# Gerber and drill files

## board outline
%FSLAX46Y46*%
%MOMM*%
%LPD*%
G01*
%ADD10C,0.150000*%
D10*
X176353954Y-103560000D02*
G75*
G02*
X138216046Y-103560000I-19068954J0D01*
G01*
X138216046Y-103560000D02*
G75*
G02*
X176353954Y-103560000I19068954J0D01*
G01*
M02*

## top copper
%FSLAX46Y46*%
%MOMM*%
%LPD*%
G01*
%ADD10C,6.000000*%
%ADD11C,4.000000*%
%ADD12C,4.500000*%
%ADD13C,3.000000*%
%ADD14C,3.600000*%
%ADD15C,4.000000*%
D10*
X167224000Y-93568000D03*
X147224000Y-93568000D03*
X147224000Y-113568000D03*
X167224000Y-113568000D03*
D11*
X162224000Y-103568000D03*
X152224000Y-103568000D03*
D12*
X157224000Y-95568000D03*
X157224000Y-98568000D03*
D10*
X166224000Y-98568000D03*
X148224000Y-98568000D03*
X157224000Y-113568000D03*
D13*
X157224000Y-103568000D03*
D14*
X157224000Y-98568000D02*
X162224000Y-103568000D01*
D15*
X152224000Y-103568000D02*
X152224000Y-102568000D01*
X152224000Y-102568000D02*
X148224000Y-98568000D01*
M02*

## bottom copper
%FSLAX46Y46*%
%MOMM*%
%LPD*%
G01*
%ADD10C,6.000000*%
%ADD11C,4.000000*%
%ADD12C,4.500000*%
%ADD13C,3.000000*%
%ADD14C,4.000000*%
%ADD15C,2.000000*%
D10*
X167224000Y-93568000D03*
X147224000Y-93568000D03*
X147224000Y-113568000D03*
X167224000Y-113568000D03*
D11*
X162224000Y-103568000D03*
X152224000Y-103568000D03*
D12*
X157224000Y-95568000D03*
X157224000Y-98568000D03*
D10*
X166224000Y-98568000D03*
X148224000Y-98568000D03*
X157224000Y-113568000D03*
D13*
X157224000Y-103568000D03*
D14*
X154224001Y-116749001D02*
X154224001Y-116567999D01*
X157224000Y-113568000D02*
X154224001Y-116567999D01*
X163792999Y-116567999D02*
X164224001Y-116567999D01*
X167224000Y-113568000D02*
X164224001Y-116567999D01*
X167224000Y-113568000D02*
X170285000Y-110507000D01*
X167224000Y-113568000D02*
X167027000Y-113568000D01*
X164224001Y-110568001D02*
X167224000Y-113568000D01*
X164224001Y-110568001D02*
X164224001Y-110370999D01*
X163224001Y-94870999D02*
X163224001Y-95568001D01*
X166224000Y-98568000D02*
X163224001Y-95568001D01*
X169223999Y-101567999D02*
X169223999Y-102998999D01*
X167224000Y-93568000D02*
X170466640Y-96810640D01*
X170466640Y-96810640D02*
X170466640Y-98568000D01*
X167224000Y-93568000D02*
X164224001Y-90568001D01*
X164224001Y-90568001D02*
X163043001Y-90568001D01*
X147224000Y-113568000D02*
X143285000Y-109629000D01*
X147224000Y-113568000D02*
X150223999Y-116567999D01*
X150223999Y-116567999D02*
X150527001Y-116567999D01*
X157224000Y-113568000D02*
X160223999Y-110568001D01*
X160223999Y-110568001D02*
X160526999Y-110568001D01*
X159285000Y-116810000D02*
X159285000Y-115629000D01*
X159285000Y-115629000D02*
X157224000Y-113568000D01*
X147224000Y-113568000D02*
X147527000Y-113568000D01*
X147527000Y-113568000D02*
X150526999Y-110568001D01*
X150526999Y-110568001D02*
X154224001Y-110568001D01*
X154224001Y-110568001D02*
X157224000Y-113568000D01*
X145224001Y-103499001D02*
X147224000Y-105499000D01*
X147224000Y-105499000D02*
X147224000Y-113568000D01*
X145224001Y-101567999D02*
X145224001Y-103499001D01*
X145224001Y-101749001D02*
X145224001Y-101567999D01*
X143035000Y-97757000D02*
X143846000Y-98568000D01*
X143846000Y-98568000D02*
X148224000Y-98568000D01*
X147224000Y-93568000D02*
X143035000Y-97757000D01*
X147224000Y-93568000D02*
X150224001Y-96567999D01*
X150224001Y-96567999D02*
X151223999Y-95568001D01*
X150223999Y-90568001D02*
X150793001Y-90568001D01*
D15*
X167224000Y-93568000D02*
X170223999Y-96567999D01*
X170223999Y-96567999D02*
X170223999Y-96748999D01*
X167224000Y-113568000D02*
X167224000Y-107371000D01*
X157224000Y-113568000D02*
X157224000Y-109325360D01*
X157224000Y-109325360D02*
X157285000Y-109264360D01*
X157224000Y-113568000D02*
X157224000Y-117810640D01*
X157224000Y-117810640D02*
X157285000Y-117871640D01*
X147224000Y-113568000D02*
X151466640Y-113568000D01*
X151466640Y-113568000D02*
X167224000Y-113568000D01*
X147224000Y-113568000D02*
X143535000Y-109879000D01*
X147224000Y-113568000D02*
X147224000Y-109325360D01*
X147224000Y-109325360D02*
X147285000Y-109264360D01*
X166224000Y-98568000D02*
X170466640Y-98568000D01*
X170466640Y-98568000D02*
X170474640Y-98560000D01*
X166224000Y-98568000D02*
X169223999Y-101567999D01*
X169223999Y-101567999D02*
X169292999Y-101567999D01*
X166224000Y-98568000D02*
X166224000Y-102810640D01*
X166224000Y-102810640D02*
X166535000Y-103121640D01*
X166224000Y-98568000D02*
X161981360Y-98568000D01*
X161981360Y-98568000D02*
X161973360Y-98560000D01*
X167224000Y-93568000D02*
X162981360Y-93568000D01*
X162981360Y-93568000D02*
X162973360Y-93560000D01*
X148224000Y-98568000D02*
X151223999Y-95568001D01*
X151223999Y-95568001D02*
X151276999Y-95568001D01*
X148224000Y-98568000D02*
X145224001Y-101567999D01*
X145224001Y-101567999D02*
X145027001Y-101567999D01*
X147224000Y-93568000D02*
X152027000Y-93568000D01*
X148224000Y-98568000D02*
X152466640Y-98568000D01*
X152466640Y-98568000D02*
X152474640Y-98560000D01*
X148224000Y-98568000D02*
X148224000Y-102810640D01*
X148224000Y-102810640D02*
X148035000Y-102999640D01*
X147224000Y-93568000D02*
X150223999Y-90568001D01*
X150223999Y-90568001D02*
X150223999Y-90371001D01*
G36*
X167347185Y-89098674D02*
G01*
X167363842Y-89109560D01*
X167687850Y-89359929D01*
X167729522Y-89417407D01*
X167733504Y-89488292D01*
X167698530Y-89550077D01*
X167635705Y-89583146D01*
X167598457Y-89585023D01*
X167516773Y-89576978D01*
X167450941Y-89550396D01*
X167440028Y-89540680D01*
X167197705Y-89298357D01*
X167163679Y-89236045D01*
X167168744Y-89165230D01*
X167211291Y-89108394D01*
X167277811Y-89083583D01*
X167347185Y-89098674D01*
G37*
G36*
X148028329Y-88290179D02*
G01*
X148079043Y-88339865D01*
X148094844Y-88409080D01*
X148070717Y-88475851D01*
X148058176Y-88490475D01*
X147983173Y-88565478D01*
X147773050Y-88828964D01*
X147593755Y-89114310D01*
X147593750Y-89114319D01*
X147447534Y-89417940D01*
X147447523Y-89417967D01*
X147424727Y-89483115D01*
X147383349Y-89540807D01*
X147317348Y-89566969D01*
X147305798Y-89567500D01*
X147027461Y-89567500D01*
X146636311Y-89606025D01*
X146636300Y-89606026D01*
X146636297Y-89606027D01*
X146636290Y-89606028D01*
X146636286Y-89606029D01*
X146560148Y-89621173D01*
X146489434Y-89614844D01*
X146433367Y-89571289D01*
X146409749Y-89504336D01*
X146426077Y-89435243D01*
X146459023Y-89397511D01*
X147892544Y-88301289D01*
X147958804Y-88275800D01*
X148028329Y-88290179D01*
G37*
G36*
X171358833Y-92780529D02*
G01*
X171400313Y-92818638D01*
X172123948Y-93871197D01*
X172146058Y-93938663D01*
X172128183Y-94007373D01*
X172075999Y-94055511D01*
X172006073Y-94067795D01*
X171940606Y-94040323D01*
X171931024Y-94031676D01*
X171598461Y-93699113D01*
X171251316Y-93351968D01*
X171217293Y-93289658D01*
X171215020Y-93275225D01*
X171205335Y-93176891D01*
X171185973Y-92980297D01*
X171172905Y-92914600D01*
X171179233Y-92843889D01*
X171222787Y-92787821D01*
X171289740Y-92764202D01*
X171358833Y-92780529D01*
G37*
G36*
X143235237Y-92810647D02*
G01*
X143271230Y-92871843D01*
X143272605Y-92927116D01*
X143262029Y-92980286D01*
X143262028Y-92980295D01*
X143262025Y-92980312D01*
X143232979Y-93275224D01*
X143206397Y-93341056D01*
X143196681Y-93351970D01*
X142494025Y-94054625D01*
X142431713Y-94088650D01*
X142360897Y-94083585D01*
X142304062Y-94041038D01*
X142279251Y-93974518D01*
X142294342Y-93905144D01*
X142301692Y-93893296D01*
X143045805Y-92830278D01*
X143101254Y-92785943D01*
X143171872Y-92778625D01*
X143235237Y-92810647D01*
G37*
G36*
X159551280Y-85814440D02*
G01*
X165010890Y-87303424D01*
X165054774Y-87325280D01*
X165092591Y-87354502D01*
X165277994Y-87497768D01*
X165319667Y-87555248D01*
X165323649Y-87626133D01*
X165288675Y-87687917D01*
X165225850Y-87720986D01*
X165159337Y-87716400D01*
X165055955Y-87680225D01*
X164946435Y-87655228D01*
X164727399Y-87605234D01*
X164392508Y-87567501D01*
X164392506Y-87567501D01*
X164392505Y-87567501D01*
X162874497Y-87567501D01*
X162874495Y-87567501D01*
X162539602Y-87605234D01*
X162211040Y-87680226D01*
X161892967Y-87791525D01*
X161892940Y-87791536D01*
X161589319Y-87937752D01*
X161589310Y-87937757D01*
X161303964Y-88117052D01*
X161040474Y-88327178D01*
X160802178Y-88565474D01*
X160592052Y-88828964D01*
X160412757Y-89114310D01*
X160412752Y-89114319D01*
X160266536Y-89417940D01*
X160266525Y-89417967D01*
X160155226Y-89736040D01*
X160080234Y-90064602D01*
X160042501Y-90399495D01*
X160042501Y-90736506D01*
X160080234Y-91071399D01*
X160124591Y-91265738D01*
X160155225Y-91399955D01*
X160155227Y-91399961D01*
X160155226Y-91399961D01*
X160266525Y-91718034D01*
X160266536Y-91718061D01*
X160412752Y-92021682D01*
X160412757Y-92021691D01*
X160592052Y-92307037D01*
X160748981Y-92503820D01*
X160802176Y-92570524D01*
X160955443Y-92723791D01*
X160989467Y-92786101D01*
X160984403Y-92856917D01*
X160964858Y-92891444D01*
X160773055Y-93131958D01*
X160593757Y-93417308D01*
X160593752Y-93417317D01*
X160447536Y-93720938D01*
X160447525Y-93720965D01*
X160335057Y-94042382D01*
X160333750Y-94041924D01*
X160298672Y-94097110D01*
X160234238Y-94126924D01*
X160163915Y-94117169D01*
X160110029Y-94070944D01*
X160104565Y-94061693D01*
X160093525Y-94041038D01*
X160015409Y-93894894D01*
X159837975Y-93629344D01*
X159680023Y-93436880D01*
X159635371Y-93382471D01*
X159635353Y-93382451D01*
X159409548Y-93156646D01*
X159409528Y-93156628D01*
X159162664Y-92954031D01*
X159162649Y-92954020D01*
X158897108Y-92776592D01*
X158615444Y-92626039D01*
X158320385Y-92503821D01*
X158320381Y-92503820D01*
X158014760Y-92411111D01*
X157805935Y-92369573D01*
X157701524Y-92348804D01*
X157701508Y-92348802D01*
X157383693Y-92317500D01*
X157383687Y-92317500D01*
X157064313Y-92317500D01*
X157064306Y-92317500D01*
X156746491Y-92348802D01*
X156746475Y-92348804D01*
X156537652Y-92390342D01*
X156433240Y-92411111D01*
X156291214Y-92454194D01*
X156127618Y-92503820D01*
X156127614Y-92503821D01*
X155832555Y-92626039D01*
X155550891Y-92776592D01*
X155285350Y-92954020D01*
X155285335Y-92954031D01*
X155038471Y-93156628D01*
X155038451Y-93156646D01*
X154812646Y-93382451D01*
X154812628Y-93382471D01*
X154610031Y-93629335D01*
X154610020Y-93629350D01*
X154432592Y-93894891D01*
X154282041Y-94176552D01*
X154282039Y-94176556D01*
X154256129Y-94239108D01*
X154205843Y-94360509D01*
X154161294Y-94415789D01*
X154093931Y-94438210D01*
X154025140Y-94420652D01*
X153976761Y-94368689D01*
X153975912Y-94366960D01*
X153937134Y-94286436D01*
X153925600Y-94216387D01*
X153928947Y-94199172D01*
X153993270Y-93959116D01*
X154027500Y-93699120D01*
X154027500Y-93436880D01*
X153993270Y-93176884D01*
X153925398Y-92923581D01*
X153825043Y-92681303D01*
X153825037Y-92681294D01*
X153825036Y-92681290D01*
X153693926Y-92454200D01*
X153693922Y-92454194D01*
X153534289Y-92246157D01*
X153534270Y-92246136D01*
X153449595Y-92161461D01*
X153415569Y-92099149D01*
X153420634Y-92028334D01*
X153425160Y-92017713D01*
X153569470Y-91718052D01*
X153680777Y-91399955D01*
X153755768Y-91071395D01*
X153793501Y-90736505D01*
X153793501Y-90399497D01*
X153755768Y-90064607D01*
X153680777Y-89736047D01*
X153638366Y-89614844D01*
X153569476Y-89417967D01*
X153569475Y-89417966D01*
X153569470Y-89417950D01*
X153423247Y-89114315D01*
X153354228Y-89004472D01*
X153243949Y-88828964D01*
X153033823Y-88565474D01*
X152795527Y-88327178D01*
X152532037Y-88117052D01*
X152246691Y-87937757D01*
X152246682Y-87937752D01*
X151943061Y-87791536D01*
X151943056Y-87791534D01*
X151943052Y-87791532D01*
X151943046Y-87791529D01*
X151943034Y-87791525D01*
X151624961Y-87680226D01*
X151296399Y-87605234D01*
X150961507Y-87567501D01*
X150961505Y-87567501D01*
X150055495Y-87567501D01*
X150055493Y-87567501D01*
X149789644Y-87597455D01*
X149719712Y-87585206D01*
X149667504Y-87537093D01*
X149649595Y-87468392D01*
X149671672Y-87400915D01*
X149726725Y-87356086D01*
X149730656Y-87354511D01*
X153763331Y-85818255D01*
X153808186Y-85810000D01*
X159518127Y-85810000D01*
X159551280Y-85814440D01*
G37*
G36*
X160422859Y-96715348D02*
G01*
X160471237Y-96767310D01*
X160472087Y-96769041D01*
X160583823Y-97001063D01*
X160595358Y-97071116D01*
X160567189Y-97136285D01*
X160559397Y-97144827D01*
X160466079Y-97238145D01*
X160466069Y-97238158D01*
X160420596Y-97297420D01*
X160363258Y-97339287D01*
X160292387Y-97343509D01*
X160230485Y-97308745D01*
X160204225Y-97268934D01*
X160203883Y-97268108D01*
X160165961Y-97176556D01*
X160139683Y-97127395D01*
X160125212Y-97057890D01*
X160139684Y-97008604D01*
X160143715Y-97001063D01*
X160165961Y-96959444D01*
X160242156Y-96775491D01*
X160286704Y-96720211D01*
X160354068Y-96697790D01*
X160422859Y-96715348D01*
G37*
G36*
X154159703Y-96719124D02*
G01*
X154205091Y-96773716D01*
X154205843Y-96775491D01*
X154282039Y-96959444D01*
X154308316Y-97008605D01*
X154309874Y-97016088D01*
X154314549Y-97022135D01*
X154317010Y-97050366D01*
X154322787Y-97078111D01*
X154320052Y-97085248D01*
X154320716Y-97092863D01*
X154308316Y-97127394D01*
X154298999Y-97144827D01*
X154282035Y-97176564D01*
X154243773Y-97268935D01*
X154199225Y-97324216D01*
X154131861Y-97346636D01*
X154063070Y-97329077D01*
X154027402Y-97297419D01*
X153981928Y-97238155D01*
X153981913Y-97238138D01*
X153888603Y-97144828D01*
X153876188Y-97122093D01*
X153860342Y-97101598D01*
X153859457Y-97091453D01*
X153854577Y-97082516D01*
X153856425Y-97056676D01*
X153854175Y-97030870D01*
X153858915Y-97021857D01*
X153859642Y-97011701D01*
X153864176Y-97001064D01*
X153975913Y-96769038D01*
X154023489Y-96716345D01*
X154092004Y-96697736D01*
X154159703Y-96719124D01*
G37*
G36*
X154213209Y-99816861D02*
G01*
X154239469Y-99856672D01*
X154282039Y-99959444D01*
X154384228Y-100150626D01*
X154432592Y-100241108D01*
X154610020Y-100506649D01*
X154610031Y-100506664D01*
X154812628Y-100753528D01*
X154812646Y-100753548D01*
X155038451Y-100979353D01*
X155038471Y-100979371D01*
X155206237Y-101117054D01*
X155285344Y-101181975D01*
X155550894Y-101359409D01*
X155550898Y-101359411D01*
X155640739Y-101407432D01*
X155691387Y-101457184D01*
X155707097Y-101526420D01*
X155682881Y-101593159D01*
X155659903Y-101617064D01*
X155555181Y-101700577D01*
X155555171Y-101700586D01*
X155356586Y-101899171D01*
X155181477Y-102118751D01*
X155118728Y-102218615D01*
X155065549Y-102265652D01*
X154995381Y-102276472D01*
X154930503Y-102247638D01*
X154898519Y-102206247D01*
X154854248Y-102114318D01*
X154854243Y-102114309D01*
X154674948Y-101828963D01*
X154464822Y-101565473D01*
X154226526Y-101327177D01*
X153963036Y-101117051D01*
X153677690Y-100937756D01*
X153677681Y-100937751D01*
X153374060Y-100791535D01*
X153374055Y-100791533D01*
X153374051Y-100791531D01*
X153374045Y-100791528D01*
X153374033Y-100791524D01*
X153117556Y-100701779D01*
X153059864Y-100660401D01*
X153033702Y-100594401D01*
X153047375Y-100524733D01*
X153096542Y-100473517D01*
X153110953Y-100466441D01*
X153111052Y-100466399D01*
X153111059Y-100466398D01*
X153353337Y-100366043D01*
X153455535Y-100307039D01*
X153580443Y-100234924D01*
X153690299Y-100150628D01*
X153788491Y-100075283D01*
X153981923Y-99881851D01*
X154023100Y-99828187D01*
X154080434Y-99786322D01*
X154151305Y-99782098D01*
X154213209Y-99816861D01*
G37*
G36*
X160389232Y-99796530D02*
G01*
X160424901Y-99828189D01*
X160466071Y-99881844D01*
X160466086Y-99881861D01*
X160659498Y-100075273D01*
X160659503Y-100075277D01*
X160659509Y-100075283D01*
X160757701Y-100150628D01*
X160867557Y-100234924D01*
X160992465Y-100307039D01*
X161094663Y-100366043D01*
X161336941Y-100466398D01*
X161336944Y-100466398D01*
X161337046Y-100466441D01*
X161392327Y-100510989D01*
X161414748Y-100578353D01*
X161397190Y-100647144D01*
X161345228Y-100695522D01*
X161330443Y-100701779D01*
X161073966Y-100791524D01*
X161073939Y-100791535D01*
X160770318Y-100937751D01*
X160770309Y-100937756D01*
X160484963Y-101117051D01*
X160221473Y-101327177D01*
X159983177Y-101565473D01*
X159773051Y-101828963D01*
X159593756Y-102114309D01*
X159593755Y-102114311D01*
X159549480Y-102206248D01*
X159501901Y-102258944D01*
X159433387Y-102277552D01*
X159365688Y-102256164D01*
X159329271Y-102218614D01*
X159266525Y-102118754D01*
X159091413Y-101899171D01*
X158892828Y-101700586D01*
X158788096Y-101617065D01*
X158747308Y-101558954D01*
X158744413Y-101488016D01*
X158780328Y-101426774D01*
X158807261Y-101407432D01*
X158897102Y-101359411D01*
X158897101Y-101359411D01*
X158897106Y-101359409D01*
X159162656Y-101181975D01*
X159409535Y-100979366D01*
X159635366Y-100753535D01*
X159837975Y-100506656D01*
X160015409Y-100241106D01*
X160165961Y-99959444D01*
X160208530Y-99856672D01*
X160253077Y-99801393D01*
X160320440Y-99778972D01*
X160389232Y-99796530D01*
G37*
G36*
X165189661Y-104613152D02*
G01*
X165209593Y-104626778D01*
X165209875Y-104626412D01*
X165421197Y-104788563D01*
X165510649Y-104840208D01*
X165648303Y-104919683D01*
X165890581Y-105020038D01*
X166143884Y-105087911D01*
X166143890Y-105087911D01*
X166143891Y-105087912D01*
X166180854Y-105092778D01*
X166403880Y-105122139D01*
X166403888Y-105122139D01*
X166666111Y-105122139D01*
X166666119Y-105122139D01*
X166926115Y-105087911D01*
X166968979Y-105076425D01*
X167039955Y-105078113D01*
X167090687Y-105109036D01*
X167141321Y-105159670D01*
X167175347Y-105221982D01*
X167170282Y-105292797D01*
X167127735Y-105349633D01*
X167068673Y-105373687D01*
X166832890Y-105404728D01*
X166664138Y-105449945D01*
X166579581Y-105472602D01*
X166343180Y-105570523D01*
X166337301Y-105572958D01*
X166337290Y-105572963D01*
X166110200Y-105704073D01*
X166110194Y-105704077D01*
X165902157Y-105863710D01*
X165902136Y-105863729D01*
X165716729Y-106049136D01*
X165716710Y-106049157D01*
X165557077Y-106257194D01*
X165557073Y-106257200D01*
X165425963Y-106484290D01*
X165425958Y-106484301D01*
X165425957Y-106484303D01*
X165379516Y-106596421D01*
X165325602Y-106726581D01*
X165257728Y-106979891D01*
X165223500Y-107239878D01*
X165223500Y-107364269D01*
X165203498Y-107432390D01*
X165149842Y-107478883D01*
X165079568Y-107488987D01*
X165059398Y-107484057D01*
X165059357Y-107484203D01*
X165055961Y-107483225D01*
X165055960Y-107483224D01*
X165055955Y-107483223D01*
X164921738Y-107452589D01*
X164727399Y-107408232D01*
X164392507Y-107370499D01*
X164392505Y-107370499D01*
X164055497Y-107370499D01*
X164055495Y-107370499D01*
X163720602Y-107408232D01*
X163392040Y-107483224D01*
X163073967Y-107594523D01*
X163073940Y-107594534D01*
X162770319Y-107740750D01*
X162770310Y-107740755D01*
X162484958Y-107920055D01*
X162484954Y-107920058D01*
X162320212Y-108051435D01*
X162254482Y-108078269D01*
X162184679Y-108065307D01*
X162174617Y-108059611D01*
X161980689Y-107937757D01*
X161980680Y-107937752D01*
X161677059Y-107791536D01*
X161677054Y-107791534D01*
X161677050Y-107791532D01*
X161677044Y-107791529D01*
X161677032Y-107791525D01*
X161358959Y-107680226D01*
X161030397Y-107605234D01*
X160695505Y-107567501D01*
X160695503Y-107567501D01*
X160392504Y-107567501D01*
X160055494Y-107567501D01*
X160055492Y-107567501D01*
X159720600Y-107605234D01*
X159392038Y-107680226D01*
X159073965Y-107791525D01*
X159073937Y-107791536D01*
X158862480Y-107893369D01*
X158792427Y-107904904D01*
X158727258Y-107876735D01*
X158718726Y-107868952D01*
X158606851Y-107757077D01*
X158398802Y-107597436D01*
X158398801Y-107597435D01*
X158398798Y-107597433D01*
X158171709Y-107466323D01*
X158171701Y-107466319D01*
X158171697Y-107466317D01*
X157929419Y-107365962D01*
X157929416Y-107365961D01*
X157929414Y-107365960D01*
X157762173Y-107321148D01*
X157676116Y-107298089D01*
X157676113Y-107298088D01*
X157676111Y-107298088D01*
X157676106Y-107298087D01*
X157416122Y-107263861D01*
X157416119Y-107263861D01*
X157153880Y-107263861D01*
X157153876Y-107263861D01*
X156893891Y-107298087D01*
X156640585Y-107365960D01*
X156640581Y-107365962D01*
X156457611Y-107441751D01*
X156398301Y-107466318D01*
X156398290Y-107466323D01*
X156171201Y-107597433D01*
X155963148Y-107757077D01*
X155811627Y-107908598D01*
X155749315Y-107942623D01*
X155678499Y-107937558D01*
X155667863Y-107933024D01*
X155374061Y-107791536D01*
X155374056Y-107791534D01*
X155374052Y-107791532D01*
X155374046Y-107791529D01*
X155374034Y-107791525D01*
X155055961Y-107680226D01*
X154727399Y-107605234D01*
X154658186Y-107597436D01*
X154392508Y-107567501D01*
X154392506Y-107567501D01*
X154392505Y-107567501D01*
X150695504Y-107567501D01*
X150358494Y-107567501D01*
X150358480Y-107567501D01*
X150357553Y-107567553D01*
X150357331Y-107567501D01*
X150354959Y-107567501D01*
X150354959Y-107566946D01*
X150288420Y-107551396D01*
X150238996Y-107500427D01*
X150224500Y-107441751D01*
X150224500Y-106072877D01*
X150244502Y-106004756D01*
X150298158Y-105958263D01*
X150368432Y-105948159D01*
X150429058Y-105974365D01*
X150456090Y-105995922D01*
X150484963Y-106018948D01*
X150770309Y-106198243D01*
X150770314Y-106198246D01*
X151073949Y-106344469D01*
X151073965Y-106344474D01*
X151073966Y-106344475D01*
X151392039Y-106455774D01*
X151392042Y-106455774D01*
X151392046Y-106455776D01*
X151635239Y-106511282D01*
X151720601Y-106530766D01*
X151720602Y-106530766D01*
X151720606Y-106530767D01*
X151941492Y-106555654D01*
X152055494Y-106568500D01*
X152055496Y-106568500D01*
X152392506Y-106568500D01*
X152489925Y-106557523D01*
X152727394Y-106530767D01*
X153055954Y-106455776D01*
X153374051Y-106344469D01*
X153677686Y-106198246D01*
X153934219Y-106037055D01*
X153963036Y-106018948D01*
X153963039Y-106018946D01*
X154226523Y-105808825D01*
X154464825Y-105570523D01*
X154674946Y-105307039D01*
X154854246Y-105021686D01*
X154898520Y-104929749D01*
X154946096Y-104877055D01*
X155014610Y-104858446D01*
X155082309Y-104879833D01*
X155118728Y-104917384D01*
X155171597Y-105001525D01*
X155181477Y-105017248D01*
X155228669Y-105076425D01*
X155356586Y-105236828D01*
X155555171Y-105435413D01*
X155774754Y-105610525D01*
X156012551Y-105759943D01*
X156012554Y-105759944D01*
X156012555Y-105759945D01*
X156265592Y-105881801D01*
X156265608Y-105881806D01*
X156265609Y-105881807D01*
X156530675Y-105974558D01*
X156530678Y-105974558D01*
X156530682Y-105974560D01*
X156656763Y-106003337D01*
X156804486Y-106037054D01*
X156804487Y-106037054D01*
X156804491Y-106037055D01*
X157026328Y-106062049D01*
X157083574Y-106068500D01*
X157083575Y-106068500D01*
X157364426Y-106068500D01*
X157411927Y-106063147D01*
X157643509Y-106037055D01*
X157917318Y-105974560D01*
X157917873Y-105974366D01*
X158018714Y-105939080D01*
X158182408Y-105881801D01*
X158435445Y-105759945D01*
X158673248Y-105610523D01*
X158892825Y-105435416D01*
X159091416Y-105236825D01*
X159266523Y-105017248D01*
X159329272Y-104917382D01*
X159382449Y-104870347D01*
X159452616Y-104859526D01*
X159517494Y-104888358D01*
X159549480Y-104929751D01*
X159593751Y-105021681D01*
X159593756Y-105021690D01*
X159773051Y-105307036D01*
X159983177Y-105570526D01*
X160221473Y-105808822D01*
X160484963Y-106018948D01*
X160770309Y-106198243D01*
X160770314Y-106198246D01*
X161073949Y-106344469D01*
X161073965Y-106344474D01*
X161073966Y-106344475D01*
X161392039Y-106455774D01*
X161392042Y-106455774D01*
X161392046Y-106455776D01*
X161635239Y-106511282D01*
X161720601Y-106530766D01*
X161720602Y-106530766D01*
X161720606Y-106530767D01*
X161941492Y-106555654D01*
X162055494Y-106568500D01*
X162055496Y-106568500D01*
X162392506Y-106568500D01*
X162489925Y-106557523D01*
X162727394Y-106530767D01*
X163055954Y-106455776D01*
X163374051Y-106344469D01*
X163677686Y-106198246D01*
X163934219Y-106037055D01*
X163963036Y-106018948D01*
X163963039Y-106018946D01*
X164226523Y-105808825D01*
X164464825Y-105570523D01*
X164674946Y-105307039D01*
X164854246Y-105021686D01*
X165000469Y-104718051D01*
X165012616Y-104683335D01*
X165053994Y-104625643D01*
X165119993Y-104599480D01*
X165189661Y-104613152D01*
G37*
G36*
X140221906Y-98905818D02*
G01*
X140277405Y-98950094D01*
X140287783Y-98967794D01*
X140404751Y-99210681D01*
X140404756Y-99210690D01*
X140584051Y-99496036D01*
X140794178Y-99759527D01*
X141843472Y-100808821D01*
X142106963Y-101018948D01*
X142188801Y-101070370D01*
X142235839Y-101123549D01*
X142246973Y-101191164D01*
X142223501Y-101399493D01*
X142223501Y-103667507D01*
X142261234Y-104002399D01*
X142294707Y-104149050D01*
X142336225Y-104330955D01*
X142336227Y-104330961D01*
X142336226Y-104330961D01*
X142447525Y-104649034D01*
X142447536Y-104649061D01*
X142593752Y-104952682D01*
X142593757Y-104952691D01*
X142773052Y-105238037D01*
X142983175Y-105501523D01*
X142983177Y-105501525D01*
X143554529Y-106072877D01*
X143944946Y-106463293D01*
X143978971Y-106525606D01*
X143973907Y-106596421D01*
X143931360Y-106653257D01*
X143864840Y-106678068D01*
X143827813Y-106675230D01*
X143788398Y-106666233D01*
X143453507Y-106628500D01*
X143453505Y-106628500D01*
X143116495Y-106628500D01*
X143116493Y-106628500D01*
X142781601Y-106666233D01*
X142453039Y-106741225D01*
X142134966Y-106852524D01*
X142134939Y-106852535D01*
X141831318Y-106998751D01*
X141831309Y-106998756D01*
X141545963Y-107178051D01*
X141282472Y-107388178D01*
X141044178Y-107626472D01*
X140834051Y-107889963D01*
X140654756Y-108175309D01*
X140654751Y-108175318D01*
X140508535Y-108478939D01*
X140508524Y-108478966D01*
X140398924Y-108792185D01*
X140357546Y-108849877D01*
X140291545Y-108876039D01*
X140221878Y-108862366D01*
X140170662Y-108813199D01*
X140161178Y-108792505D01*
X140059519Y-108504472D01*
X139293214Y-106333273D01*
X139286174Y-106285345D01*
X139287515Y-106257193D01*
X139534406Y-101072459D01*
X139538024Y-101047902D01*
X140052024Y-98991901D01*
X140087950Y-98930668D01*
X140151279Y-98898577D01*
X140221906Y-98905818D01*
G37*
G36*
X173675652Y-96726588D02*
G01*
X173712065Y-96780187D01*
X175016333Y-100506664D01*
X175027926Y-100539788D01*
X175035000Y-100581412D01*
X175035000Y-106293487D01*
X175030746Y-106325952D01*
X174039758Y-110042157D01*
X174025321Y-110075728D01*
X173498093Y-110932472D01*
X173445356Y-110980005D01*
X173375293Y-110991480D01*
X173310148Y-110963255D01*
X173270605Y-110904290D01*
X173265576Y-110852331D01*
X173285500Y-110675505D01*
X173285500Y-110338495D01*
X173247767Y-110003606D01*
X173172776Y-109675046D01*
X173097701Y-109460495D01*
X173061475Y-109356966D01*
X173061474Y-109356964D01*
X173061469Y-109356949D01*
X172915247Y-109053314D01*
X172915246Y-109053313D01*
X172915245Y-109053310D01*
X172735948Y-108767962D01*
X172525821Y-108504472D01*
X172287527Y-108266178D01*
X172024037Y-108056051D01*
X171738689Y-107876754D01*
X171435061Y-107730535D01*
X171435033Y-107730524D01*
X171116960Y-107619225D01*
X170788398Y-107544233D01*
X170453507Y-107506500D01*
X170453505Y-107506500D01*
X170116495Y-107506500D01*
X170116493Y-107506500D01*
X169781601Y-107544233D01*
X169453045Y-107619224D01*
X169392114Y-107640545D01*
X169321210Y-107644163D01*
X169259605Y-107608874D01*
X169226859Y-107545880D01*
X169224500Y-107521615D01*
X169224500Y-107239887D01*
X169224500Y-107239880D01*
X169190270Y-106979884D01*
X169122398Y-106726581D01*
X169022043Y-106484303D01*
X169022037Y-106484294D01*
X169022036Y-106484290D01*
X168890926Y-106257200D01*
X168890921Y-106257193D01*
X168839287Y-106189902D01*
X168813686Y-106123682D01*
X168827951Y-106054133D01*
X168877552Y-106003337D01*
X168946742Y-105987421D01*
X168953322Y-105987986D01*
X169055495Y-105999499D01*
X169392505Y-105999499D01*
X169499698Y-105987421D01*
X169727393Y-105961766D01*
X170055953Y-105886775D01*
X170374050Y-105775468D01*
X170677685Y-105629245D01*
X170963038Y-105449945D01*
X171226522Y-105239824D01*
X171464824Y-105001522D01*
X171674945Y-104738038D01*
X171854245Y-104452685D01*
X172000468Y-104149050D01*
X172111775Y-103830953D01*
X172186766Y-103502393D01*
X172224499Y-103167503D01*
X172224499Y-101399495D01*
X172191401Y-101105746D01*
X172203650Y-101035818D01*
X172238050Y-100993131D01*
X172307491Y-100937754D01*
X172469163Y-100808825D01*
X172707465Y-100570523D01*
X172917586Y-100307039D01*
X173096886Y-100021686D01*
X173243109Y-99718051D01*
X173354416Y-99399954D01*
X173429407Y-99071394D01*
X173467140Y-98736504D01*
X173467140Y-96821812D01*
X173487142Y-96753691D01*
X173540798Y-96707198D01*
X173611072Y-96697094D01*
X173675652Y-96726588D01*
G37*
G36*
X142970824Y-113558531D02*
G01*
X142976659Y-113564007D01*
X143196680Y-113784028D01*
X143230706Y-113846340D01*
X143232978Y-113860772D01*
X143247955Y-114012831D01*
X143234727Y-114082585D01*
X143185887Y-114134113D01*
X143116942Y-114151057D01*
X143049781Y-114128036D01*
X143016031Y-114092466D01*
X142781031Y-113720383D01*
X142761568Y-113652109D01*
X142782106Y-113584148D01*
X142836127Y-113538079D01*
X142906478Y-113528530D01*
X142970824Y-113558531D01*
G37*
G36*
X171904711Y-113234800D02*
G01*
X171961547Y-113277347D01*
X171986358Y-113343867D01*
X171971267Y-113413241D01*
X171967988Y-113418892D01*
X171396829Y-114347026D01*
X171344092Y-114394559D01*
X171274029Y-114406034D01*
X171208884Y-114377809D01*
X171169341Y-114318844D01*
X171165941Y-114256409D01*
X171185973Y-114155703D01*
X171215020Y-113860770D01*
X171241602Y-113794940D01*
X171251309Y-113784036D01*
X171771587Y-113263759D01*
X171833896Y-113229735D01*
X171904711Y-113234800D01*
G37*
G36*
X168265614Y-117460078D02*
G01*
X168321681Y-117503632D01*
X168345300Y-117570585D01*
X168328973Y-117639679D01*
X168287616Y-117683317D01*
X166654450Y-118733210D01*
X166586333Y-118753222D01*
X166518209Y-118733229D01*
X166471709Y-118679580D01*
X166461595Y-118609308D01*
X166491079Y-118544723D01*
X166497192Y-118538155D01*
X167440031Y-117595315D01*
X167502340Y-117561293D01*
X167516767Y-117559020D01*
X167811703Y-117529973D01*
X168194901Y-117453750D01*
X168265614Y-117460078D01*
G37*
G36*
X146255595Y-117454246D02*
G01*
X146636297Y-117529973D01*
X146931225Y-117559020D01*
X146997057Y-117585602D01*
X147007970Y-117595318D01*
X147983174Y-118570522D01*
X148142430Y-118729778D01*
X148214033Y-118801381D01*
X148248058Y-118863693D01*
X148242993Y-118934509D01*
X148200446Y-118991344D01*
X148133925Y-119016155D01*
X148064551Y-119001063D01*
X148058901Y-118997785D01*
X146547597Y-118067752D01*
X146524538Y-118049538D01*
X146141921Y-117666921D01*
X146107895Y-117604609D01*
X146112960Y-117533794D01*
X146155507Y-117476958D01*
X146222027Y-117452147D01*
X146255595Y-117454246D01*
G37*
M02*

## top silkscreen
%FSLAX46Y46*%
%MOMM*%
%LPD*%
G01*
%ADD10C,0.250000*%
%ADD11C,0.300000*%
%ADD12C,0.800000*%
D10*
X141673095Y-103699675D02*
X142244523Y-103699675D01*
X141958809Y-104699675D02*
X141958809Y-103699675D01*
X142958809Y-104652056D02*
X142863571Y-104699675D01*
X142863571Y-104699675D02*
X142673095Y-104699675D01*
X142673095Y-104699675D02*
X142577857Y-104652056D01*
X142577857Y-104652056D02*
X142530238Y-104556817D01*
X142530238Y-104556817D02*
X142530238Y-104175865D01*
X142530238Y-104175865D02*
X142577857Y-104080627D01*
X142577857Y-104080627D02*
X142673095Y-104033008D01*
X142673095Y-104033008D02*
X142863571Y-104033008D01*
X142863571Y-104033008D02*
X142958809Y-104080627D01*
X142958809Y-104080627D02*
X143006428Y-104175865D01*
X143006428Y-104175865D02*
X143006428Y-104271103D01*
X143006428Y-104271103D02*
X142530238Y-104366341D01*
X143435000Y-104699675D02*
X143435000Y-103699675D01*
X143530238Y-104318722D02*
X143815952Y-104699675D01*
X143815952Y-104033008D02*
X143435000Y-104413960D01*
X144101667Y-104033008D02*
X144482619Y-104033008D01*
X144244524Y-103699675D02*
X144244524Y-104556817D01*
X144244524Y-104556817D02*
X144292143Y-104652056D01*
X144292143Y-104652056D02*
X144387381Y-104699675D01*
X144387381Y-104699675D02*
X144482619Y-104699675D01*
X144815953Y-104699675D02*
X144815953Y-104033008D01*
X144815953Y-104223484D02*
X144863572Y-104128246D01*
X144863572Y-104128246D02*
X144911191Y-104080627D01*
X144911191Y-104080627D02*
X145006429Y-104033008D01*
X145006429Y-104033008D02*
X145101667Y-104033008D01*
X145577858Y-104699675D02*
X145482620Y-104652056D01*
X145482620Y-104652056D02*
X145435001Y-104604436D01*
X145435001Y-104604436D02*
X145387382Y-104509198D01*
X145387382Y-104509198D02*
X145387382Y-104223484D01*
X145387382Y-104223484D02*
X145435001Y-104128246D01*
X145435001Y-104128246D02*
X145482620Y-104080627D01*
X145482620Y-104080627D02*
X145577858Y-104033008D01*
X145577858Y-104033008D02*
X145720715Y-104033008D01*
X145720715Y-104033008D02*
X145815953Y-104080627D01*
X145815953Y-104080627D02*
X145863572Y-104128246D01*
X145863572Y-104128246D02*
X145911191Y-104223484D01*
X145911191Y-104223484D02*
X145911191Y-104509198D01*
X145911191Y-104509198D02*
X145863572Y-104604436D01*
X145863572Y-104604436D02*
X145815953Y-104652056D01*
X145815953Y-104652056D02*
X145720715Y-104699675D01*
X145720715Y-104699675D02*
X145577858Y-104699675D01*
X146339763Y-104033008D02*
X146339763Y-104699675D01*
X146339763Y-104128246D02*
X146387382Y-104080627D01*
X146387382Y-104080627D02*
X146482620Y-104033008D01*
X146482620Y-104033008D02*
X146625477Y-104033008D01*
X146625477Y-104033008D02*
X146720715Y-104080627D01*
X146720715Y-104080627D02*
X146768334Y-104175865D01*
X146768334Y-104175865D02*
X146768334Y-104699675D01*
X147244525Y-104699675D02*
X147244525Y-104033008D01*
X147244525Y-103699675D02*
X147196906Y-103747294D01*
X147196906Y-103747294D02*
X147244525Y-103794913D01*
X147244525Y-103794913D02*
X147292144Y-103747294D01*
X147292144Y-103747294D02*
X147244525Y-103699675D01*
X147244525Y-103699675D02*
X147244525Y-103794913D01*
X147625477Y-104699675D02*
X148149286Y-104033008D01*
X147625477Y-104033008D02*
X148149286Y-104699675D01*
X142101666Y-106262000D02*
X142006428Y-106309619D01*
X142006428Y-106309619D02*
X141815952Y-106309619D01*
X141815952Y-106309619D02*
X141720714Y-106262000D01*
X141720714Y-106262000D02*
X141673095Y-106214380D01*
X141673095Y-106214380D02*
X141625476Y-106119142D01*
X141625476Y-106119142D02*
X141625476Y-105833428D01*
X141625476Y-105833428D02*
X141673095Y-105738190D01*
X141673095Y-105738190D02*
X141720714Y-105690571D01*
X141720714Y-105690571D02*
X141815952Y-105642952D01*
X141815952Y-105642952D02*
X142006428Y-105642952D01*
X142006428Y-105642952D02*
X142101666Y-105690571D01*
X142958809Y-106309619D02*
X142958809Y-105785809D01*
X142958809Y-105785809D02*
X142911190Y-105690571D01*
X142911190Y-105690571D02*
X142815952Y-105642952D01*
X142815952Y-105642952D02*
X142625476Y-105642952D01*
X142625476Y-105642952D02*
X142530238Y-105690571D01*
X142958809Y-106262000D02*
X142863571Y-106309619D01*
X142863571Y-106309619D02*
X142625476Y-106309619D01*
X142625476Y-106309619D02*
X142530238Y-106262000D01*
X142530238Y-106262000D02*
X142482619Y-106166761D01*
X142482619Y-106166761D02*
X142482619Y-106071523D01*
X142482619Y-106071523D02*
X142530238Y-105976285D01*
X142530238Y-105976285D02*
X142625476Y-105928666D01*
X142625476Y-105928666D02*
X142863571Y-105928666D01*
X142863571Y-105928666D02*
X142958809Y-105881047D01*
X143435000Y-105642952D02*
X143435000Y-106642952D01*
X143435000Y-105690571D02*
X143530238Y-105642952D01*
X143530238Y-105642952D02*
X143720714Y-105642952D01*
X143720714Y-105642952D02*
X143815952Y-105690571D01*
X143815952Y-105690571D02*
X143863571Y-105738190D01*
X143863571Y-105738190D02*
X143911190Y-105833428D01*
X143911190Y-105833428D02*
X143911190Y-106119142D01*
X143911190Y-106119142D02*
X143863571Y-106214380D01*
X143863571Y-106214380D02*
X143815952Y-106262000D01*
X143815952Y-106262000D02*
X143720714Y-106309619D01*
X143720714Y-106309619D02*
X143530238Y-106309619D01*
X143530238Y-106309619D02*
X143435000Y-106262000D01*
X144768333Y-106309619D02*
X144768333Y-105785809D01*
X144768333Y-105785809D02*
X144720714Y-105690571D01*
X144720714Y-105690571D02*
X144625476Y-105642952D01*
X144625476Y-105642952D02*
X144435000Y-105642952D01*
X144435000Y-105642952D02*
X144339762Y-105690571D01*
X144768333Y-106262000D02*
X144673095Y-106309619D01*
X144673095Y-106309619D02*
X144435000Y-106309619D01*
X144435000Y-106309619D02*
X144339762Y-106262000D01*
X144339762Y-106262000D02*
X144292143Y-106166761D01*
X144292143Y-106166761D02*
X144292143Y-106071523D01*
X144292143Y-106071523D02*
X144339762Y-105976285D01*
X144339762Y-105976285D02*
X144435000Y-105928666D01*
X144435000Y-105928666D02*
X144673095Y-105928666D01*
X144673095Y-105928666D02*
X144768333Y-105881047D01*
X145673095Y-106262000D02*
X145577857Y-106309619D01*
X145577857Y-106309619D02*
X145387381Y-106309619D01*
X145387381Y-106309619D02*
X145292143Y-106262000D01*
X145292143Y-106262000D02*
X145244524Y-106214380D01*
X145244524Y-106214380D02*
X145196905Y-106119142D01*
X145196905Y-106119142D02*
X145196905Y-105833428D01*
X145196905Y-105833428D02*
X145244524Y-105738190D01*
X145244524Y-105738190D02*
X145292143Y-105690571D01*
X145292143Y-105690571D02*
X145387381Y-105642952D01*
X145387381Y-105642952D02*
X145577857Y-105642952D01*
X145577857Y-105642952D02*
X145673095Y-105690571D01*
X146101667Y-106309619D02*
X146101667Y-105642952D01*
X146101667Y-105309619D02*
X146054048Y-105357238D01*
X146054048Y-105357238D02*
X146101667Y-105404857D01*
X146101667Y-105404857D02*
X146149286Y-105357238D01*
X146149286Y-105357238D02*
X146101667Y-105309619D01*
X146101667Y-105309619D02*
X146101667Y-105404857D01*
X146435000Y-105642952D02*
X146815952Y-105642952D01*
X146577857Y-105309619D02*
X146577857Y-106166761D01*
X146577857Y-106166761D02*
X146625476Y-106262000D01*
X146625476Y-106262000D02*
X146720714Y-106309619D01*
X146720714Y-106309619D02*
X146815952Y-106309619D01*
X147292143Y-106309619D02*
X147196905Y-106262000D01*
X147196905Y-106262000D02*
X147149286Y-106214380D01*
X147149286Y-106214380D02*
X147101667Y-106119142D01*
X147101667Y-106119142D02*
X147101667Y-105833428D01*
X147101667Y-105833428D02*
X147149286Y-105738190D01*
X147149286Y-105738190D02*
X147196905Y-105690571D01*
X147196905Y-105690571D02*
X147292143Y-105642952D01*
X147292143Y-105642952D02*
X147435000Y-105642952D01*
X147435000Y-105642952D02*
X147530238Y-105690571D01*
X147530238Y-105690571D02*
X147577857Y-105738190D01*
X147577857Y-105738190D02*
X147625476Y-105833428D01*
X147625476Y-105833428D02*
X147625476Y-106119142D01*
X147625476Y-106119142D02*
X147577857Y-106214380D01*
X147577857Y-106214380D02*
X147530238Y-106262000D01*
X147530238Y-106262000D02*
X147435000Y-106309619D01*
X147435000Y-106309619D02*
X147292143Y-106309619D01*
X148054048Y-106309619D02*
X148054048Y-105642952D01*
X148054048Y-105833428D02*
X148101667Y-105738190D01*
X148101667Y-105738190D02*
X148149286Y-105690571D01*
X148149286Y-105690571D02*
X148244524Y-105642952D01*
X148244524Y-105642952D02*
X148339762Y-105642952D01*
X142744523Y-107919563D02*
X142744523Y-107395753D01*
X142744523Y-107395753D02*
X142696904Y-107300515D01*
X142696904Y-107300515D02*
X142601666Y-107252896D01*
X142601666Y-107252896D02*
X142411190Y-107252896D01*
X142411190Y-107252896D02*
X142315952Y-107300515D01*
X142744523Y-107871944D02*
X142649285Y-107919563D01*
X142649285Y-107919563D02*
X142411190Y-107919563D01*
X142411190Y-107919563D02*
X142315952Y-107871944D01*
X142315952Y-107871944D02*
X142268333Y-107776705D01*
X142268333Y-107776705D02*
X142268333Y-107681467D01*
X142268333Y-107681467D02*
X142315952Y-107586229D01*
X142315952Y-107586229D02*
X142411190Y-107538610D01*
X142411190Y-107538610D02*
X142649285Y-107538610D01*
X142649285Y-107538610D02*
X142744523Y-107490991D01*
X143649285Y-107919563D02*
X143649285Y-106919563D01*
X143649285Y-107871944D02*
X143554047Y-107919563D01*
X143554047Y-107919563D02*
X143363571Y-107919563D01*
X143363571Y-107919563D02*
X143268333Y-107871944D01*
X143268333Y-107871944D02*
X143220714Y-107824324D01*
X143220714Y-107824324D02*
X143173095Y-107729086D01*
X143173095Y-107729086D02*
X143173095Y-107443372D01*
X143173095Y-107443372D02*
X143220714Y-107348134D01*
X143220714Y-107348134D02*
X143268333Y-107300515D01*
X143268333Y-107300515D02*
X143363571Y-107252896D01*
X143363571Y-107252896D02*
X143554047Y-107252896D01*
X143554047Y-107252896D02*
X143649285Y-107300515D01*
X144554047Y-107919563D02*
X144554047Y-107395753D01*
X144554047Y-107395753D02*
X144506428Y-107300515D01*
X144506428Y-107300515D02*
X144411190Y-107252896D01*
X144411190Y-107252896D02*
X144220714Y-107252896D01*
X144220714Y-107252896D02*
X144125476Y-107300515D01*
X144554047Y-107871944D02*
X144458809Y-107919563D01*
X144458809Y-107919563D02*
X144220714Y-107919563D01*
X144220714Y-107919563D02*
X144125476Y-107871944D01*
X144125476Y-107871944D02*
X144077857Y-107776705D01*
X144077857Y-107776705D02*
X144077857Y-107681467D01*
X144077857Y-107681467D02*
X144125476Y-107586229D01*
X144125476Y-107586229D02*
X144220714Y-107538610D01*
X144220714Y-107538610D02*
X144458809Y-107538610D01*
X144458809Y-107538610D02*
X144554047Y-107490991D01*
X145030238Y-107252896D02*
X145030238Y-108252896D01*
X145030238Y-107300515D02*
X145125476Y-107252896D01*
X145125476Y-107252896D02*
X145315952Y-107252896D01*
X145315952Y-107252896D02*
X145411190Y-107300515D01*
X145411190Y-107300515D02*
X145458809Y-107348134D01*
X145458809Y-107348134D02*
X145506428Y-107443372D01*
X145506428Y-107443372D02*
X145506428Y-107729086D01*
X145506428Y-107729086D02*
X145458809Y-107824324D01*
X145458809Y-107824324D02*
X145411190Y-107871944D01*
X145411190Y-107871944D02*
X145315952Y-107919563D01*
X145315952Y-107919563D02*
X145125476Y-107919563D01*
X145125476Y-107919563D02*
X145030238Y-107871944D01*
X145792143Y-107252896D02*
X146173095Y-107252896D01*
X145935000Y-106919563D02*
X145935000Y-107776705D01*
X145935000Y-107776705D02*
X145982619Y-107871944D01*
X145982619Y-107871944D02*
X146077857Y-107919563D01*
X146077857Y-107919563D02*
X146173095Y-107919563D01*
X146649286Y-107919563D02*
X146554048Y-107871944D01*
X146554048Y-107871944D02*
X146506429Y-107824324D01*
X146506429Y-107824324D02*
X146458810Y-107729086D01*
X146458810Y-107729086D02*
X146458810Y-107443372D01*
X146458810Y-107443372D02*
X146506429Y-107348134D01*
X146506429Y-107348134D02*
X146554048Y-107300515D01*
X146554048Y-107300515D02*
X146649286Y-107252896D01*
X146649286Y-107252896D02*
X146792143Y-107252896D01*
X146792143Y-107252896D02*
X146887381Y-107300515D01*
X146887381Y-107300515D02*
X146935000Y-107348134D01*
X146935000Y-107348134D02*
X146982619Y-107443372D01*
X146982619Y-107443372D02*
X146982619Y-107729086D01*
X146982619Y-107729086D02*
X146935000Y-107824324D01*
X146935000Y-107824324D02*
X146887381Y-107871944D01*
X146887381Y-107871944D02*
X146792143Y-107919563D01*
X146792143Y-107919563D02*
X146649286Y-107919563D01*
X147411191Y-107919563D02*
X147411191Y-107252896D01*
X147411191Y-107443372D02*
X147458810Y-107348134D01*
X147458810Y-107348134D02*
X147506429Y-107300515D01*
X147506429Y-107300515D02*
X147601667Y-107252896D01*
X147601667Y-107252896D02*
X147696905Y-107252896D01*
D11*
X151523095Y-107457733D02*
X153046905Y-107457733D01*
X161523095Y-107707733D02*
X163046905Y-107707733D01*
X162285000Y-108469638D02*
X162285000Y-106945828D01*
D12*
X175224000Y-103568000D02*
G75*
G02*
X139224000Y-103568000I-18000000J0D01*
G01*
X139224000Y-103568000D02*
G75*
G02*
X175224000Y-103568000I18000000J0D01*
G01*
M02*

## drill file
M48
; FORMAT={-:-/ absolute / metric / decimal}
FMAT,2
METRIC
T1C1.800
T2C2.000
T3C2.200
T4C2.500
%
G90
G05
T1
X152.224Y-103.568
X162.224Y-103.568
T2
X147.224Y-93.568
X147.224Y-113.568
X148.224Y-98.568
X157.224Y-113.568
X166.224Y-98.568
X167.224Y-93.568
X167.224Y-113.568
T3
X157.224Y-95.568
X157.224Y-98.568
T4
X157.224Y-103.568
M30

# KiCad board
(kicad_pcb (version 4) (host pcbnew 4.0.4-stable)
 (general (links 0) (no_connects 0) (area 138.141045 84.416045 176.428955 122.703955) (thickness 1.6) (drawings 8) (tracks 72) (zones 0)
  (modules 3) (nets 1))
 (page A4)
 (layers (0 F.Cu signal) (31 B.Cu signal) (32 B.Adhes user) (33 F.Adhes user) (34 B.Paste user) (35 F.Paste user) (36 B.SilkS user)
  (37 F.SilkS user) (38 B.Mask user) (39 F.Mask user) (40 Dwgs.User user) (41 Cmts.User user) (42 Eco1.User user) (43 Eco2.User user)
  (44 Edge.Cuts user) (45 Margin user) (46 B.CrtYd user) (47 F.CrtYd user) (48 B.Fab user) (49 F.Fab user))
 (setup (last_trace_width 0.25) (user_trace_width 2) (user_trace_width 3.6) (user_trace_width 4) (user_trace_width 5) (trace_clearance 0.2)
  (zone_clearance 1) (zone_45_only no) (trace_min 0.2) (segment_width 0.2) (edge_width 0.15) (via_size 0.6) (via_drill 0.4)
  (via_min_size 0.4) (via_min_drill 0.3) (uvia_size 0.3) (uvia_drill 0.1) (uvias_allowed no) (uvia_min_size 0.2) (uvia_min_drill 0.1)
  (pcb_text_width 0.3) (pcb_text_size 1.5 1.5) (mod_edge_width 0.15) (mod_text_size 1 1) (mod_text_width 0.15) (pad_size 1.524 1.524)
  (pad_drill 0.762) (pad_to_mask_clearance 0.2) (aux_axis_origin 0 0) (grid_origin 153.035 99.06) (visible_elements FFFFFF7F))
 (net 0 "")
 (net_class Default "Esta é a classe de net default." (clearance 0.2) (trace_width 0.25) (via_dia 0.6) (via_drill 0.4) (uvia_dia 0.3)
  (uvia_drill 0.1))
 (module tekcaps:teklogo (layer B.Cu) (at 169.535 105.16 180)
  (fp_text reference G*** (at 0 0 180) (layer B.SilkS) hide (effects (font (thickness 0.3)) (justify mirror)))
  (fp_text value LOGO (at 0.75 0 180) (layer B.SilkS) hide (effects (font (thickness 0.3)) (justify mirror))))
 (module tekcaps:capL (layer F.Cu) (at 157.224 103.568)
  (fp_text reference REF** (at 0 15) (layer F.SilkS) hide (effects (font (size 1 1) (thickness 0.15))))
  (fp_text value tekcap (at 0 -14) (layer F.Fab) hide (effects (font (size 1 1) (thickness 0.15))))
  (fp_circle (center 0 0) (end 18 0) (layer F.SilkS) (width 0.8))
  (pad 1 thru_hole circle (at 10 -10) (size 6 6) (drill 2) (layers *.Cu *.Mask))
  (pad 1 thru_hole circle (at -10 -10) (size 6 6) (drill 2) (layers *.Cu *.Mask))
  (pad 1 thru_hole circle (at -10 10) (size 6 6) (drill 2) (layers *.Cu *.Mask))
  (pad 1 thru_hole circle (at 10 10) (size 6 6) (drill 2) (layers *.Cu *.Mask))
  (pad 2 thru_hole circle (at 5 0) (size 4 4) (drill 1.8) (layers *.Cu *.Mask))
  (pad 1 thru_hole circle (at -5 0) (size 4 4) (drill 1.8) (layers *.Cu *.Mask))
  (pad 2 thru_hole circle (at 0 -8) (size 4.5 4.5) (drill 2.2) (layers *.Cu *.Mask))
  (pad 2 thru_hole circle (at 0 -5) (size 4.5 4.5) (drill 2.2) (layers *.Cu *.Mask))
  (pad 1 thru_hole circle (at 9 -5) (size 6 6) (drill 2) (layers *.Cu *.Mask))
  (pad 1 thru_hole circle (at -9 -5) (size 6 6) (drill 2) (layers *.Cu *.Mask))
  (pad 1 thru_hole circle (at 0 10) (size 6 6) (drill 2) (layers *.Cu *.Mask))
  (pad "" np_thru_hole circle (at 0 0) (size 3 3) (drill 2.5) (layers *.Cu *.Mask)))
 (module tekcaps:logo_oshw (layer B.Cu) (at 145.735 105.86 180)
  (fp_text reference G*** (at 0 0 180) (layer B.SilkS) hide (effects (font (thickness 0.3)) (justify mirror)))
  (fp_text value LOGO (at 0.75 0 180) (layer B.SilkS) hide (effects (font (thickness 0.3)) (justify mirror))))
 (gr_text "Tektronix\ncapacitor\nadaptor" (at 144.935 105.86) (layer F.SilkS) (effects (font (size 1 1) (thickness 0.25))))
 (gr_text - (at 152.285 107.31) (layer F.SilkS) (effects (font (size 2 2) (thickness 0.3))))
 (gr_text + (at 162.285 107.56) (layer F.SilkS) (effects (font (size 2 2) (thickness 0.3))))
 (gr_circle (center 157.285 103.56) (end 173.035 114.31) (layer Edge.Cuts) (width 0.15))
 (segment (start 157.224 98.568) (end 162.224 103.568) (width 3.6) (layer F.Cu) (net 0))
 (segment (start 152.224 103.568) (end 152.224 102.568) (width 4) (layer F.Cu) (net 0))
 (segment (start 152.224 102.568) (end 148.224 98.568) (width 4) (layer F.Cu) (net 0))
 (segment (start 154.224001 116.749001) (end 154.224001 116.567999) (width 4) (layer B.Cu) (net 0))
 (segment (start 157.224 113.568) (end 154.224001 116.567999) (width 4) (layer B.Cu) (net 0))
 (segment (start 163.792999 116.567999) (end 164.224001 116.567999) (width 4) (layer B.Cu) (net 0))
 (segment (start 167.224 113.568) (end 164.224001 116.567999) (width 4) (layer B.Cu) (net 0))
 (segment (start 167.224 113.568) (end 170.285 110.507) (width 4) (layer B.Cu) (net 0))
 (segment (start 167.224 113.568) (end 167.027 113.568) (width 4) (layer B.Cu) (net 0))
 (segment (start 164.224001 110.568001) (end 167.224 113.568) (width 4) (layer B.Cu) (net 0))
 (segment (start 164.224001 110.568001) (end 164.224001 110.370999) (width 4) (layer B.Cu) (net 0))
 (segment (start 163.224001 94.870999) (end 163.224001 95.568001) (width 4) (layer B.Cu) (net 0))
 (segment (start 166.224 98.568) (end 163.224001 95.568001) (width 4) (layer B.Cu) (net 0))
 (segment (start 169.223999 101.567999) (end 169.223999 102.998999) (width 4) (layer B.Cu) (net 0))
 (segment (start 167.224 93.568) (end 170.46664 96.81064) (width 4) (layer B.Cu) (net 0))
 (segment (start 170.46664 96.81064) (end 170.46664 98.568) (width 4) (layer B.Cu) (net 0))
 (segment (start 167.224 93.568) (end 164.224001 90.568001) (width 4) (layer B.Cu) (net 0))
 (segment (start 164.224001 90.568001) (end 163.043001 90.568001) (width 4) (layer B.Cu) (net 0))
 (segment (start 147.224 113.568) (end 143.285 109.629) (width 4) (layer B.Cu) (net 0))
 (segment (start 147.224 113.568) (end 150.223999 116.567999) (width 4) (layer B.Cu) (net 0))
 (segment (start 150.223999 116.567999) (end 150.527001 116.567999) (width 4) (layer B.Cu) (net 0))
 (segment (start 157.224 113.568) (end 160.223999 110.568001) (width 4) (layer B.Cu) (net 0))
 (segment (start 160.223999 110.568001) (end 160.526999 110.568001) (width 4) (layer B.Cu) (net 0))
 (segment (start 159.285 116.81) (end 159.285 115.629) (width 4) (layer B.Cu) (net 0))
 (segment (start 159.285 115.629) (end 157.224 113.568) (width 4) (layer B.Cu) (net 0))
 (segment (start 147.224 113.568) (end 147.527 113.568) (width 4) (layer B.Cu) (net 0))
 (segment (start 147.527 113.568) (end 150.526999 110.568001) (width 4) (layer B.Cu) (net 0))
 (segment (start 150.526999 110.568001) (end 154.224001 110.568001) (width 4) (layer B.Cu) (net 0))
 (segment (start 154.224001 110.568001) (end 157.224 113.568) (width 4) (layer B.Cu) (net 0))
 (segment (start 145.224001 103.499001) (end 147.224 105.499) (width 4) (layer B.Cu) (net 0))
 (segment (start 147.224 105.499) (end 147.224 113.568) (width 4) (layer B.Cu) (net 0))
 (segment (start 145.224001 101.567999) (end 145.224001 103.499001) (width 4) (layer B.Cu) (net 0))
 (segment (start 145.224001 101.749001) (end 145.224001 101.567999) (width 4) (layer B.Cu) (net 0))
 (segment (start 143.035 97.757) (end 143.846 98.568) (width 4) (layer B.Cu) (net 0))
 (segment (start 143.846 98.568) (end 148.224 98.568) (width 4) (layer B.Cu) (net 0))
 (segment (start 147.224 93.568) (end 143.035 97.757) (width 4) (layer B.Cu) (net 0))
 (segment (start 147.224 93.568) (end 150.224001 96.567999) (width 4) (layer B.Cu) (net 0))
 (segment (start 150.224001 96.567999) (end 151.223999 95.568001) (width 4) (layer B.Cu) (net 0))
 (segment (start 150.223999 90.568001) (end 150.793001 90.568001) (width 4) (layer B.Cu) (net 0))
 (segment (start 167.224 93.568) (end 170.223999 96.567999) (width 2) (layer B.Cu) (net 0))
 (segment (start 170.223999 96.567999) (end 170.223999 96.748999) (width 2) (layer B.Cu) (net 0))
 (segment (start 167.224 113.568) (end 167.224 107.371) (width 2) (layer B.Cu) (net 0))
 (segment (start 157.224 113.568) (end 157.224 109.32536) (width 2) (layer B.Cu) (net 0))
 (segment (start 157.224 109.32536) (end 157.285 109.26436) (width 2) (layer B.Cu) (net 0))
 (segment (start 157.224 113.568) (end 157.224 117.81064) (width 2) (layer B.Cu) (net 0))
 (segment (start 157.224 117.81064) (end 157.285 117.87164) (width 2) (layer B.Cu) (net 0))
 (segment (start 147.224 113.568) (end 151.46664 113.568) (width 2) (layer B.Cu) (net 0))
 (segment (start 151.46664 113.568) (end 167.224 113.568) (width 2) (layer B.Cu) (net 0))
 (segment (start 147.224 113.568) (end 143.535 109.879) (width 2) (layer B.Cu) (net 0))
 (segment (start 147.224 113.568) (end 147.224 109.32536) (width 2) (layer B.Cu) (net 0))
 (segment (start 147.224 109.32536) (end 147.285 109.26436) (width 2) (layer B.Cu) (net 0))
 (segment (start 166.224 98.568) (end 170.46664 98.568) (width 2) (layer B.Cu) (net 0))
 (segment (start 170.46664 98.568) (end 170.47464 98.56) (width 2) (layer B.Cu) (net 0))
 (segment (start 166.224 98.568) (end 169.223999 101.567999) (width 2) (layer B.Cu) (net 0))
 (segment (start 169.223999 101.567999) (end 169.292999 101.567999) (width 2) (layer B.Cu) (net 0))
 (segment (start 166.224 98.568) (end 166.224 102.81064) (width 2) (layer B.Cu) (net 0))
 (segment (start 166.224 102.81064) (end 166.535 103.12164) (width 2) (layer B.Cu) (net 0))
 (segment (start 166.224 98.568) (end 161.98136 98.568) (width 2) (layer B.Cu) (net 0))
 (segment (start 161.98136 98.568) (end 161.97336 98.56) (width 2) (layer B.Cu) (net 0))
 (segment (start 167.224 93.568) (end 162.98136 93.568) (width 2) (layer B.Cu) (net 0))
 (segment (start 162.98136 93.568) (end 162.97336 93.56) (width 2) (layer B.Cu) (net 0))
 (segment (start 148.224 98.568) (end 151.223999 95.568001) (width 2) (layer B.Cu) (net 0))
 (segment (start 151.223999 95.568001) (end 151.276999 95.568001) (width 2) (layer B.Cu) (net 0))
 (segment (start 148.224 98.568) (end 145.224001 101.567999) (width 2) (layer B.Cu) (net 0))
 (segment (start 145.224001 101.567999) (end 145.027001 101.567999) (width 2) (layer B.Cu) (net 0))
 (segment (start 147.224 93.568) (end 152.027 93.568) (width 2) (layer B.Cu) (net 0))
 (segment (start 148.224 98.568) (end 152.46664 98.568) (width 2) (layer B.Cu) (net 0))
 (segment (start 152.46664 98.568) (end 152.47464 98.56) (width 2) (layer B.Cu) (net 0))
 (segment (start 148.224 98.568) (end 148.224 102.81064) (width 2) (layer B.Cu) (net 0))
 (segment (start 148.224 102.81064) (end 148.035 102.99964) (width 2) (layer B.Cu) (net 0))
 (segment (start 147.224 93.568) (end 150.223999 90.568001) (width 2) (layer B.Cu) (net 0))
 (segment (start 150.223999 90.568001) (end 150.223999 90.371001) (width 2) (layer B.Cu) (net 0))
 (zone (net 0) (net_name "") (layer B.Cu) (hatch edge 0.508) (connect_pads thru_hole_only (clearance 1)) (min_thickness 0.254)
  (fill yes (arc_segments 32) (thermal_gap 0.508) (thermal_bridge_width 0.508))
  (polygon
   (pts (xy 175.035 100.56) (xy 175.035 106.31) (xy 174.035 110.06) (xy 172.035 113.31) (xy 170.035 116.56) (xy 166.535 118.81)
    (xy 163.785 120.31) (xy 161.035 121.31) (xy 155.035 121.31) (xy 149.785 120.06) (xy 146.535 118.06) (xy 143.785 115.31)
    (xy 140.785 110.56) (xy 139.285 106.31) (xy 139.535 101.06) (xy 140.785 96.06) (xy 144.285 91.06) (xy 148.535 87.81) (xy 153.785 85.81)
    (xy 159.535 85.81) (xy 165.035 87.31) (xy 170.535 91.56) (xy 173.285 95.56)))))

